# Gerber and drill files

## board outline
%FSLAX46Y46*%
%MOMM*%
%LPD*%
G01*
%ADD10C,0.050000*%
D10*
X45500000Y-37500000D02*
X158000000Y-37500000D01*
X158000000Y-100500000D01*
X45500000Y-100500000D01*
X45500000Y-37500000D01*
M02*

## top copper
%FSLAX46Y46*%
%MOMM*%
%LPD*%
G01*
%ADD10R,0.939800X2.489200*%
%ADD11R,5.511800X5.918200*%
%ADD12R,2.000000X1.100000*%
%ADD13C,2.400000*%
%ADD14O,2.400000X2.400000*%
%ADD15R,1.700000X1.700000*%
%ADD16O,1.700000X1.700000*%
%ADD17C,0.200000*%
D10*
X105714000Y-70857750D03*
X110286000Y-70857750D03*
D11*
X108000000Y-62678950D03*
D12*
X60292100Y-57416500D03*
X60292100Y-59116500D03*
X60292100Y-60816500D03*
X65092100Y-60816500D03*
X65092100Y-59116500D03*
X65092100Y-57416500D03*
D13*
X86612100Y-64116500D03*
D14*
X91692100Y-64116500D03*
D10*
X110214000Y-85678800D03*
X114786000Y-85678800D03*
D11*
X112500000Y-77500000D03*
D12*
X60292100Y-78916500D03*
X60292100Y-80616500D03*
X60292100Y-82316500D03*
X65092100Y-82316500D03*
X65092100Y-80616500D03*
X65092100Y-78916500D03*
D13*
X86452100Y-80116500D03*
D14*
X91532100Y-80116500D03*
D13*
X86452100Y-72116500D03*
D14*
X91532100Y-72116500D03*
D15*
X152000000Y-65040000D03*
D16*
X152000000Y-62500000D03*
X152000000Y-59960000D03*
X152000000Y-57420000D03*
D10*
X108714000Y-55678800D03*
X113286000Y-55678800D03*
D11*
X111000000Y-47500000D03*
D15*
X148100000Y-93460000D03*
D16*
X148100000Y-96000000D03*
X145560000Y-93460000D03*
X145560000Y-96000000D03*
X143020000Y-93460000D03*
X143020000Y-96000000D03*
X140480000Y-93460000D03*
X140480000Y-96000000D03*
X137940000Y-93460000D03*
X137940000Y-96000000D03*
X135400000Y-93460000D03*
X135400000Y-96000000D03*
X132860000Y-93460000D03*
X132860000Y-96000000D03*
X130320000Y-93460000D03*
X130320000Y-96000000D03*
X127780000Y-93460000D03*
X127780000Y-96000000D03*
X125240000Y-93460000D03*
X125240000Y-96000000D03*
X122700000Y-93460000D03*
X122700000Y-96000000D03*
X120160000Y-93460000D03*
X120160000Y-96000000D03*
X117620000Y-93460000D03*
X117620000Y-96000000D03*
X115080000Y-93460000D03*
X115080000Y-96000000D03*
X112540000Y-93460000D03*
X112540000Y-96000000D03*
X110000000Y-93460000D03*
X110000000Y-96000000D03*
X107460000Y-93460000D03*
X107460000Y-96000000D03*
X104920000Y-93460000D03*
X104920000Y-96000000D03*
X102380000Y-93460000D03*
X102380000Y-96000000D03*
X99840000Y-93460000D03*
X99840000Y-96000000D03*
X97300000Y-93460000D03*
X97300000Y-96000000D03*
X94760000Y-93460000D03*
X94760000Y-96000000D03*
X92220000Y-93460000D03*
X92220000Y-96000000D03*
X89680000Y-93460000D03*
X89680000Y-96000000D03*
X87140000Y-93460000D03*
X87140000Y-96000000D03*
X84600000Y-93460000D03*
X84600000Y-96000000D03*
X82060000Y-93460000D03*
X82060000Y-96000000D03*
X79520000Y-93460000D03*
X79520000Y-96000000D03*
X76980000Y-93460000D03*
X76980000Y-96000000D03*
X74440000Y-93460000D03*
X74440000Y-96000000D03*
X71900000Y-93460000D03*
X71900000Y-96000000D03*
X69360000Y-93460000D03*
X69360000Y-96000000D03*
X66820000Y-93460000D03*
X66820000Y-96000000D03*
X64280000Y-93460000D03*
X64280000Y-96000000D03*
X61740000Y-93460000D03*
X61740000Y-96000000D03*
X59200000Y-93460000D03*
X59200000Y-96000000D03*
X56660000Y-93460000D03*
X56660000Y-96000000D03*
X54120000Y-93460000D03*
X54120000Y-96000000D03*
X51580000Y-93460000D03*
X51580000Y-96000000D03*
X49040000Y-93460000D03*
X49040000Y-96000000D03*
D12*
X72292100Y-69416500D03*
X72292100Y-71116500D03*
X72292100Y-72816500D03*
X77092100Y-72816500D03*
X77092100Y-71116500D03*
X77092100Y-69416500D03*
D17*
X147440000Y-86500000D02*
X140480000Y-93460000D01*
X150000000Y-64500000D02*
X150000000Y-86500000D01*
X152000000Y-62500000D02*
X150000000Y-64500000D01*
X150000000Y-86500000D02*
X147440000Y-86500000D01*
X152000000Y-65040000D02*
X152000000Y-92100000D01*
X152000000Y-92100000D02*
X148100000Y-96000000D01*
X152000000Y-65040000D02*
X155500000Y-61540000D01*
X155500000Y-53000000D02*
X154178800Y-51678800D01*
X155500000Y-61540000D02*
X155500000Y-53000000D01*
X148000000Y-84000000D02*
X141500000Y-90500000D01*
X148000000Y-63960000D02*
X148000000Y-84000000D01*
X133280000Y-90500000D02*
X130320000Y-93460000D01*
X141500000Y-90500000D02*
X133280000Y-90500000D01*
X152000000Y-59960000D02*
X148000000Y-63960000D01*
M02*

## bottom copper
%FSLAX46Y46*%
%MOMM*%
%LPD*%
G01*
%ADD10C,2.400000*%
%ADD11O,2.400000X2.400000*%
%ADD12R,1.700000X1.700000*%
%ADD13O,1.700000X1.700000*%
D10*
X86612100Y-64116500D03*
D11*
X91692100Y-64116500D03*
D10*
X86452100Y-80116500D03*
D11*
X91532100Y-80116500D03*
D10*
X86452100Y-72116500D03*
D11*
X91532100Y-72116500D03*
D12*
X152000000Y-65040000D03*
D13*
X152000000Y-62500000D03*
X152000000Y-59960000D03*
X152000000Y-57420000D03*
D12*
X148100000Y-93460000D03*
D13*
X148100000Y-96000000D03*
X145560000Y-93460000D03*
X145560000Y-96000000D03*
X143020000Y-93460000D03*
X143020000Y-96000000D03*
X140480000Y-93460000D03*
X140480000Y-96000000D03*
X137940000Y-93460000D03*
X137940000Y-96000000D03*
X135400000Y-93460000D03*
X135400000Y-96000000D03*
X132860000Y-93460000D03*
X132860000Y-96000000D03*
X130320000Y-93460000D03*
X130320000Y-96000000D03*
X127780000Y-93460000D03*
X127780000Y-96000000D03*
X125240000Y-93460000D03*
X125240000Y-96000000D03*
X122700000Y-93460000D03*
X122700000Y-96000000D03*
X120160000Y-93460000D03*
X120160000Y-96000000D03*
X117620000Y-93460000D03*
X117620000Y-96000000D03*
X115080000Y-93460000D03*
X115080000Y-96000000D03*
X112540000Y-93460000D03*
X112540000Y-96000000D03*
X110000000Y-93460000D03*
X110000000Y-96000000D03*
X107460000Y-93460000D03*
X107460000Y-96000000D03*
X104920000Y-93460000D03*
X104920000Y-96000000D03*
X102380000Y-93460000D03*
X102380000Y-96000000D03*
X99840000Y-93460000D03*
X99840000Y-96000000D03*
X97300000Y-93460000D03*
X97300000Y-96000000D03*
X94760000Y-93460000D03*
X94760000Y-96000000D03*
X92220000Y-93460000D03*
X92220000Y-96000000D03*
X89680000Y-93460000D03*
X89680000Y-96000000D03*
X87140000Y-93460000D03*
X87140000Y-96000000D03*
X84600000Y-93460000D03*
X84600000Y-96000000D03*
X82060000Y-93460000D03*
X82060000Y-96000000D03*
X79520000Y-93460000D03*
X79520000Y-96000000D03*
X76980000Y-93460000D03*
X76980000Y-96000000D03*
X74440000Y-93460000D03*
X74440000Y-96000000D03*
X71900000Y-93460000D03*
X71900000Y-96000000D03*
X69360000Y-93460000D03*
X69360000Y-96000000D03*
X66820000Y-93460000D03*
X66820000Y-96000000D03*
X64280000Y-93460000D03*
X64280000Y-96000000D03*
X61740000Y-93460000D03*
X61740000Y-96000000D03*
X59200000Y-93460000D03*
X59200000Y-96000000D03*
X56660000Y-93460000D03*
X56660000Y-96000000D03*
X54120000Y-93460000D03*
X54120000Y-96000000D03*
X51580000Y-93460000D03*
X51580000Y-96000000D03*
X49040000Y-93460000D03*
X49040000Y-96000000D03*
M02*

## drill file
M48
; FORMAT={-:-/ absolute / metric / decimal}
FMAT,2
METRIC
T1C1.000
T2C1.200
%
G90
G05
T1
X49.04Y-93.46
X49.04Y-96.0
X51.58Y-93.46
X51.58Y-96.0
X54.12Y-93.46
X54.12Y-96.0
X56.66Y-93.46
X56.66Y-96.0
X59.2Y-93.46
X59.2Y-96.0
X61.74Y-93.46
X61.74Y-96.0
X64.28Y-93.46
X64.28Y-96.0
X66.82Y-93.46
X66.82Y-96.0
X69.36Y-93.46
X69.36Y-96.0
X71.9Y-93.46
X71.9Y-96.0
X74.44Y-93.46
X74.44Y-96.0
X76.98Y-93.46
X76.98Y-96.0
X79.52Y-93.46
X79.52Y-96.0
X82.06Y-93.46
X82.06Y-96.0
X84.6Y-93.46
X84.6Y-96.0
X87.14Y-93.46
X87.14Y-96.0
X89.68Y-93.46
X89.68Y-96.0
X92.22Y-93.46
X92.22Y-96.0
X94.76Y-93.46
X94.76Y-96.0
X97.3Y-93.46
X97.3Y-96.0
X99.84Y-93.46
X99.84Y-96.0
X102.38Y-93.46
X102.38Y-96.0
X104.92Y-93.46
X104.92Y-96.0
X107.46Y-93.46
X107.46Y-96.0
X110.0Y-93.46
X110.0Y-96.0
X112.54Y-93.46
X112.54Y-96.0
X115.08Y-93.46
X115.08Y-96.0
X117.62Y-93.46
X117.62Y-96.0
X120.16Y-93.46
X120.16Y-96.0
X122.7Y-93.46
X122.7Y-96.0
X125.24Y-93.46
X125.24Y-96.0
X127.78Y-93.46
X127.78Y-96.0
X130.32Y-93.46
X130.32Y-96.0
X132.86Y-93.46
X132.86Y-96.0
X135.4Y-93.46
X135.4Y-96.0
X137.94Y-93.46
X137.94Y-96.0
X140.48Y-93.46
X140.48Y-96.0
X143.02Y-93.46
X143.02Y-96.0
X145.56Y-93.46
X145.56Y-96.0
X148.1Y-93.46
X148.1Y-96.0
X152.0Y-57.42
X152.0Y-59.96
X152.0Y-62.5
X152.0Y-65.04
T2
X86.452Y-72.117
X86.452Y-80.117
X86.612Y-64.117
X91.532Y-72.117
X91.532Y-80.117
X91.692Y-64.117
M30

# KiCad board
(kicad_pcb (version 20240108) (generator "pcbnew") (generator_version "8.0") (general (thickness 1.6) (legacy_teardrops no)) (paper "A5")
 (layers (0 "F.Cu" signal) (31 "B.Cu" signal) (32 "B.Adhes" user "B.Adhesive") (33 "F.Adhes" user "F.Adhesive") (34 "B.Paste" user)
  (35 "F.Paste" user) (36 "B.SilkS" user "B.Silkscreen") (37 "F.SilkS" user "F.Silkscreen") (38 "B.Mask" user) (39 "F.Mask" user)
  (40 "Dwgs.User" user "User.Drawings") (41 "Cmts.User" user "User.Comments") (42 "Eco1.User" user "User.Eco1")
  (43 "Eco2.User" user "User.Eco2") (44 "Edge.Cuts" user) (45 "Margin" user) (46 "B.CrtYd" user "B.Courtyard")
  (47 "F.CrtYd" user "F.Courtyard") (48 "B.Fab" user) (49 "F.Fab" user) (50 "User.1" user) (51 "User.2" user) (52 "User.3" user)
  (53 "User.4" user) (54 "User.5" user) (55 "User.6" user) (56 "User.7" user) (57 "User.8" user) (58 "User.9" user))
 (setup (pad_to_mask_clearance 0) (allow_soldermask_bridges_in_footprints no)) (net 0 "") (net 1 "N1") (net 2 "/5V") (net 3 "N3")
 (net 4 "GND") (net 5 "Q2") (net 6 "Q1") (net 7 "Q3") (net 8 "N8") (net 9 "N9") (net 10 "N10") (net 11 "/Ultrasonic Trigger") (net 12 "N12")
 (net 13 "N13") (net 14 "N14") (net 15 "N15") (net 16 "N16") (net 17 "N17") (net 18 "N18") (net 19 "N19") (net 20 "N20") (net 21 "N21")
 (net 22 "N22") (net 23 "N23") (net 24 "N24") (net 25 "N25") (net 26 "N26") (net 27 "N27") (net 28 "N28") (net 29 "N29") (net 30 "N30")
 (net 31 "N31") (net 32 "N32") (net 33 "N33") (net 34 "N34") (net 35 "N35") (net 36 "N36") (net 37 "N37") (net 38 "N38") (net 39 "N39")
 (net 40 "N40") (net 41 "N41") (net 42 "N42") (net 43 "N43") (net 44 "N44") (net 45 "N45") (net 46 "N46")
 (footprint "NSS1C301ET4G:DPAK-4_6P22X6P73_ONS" (layer "F.Cu") (at 108 64.44425)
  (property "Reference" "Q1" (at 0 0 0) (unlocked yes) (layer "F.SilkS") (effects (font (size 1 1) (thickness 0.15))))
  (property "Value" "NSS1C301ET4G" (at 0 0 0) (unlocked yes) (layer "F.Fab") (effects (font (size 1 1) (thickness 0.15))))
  (pad "1" smd rect (at -2.286 6.4135) (size 0.9398 2.4892) (layers "F.Cu" "F.Paste" "F.Mask") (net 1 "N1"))
  (pad "2" smd rect (at 2.286 6.4135) (size 0.9398 2.4892) (layers "F.Cu" "F.Paste" "F.Mask") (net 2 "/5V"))
  (pad "3" smd rect (at 0 -1.7653) (size 5.5118 5.9182) (layers "F.Cu" "F.Paste" "F.Mask") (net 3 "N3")))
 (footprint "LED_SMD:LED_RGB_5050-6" (layer "F.Cu") (at 62.6921 59.1165)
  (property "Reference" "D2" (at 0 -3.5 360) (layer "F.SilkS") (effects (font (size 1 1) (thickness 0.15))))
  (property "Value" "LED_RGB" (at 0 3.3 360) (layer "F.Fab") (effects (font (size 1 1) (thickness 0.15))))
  (pad "1" smd rect (at -2.4 -1.7 90) (size 1.1 2) (layers "F.Cu" "F.Paste" "F.Mask") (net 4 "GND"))
  (pad "2" smd rect (at -2.4 0 90) (size 1.1 2) (layers "F.Cu" "F.Paste" "F.Mask") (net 4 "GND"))
  (pad "3" smd rect (at -2.4 1.7 90) (size 1.1 2) (layers "F.Cu" "F.Paste" "F.Mask") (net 4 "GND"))
  (pad "4" smd rect (at 2.4 1.7 90) (size 1.1 2) (layers "F.Cu" "F.Paste" "F.Mask") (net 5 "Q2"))
  (pad "5" smd rect (at 2.4 0 90) (size 1.1 2) (layers "F.Cu" "F.Paste" "F.Mask") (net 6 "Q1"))
  (pad "6" smd rect (at 2.4 -1.7 90) (size 1.1 2) (layers "F.Cu" "F.Paste" "F.Mask") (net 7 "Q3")))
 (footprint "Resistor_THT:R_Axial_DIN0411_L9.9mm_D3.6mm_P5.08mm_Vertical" (layer "F.Cu") (at 86.6121 64.1165)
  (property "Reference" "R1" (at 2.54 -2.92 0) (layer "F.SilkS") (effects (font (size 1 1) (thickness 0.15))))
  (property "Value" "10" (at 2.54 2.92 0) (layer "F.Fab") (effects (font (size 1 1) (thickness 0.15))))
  (pad "1" thru_hole circle (at 0 0) (size 2.4 2.4) (drill 1.2) (layers "*.Cu" "*.Mask") (remove_unused_layers no) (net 7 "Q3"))
  (pad "2" thru_hole oval (at 5.08 0) (size 2.4 2.4) (drill 1.2) (layers "*.Cu" "*.Mask") (remove_unused_layers no) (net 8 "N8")))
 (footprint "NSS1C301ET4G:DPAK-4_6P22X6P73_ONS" (layer "F.Cu") (at 112.5 79.2653)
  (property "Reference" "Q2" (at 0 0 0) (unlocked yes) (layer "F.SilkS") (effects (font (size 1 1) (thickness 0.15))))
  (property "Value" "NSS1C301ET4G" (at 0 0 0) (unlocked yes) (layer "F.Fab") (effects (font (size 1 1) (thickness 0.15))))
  (pad "1" smd rect (at -2.286 6.4135) (size 0.9398 2.4892) (layers "F.Cu" "F.Paste" "F.Mask") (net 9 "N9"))
  (pad "2" smd rect (at 2.286 6.4135) (size 0.9398 2.4892) (layers "F.Cu" "F.Paste" "F.Mask") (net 2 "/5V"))
  (pad "3" smd rect (at 0 -1.7653) (size 5.5118 5.9182) (layers "F.Cu" "F.Paste" "F.Mask") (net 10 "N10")))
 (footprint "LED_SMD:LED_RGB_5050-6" (layer "F.Cu") (at 62.6921 80.6165)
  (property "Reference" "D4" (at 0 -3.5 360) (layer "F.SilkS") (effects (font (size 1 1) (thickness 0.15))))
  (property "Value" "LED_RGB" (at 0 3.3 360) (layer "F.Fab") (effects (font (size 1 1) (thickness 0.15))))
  (pad "1" smd rect (at -2.4 -1.7 90) (size 1.1 2) (layers "F.Cu" "F.Paste" "F.Mask") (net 4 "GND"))
  (pad "2" smd rect (at -2.4 0 90) (size 1.1 2) (layers "F.Cu" "F.Paste" "F.Mask") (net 4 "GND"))
  (pad "3" smd rect (at -2.4 1.7 90) (size 1.1 2) (layers "F.Cu" "F.Paste" "F.Mask") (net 4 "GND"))
  (pad "4" smd rect (at 2.4 1.7 90) (size 1.1 2) (layers "F.Cu" "F.Paste" "F.Mask") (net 5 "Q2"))
  (pad "5" smd rect (at 2.4 0 90) (size 1.1 2) (layers "F.Cu" "F.Paste" "F.Mask") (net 6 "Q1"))
  (pad "6" smd rect (at 2.4 -1.7 90) (size 1.1 2) (layers "F.Cu" "F.Paste" "F.Mask") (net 7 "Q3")))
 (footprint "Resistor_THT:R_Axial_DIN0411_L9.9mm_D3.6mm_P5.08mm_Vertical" (layer "F.Cu") (at 86.4521 80.1165)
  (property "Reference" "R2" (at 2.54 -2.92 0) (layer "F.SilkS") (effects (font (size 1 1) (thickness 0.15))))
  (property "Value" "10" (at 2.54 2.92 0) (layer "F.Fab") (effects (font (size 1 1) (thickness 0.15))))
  (pad "1" thru_hole circle (at 0 0) (size 2.4 2.4) (drill 1.2) (layers "*.Cu" "*.Mask") (remove_unused_layers no) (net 5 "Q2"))
  (pad "2" thru_hole oval (at 5.08 0) (size 2.4 2.4) (drill 1.2) (layers "*.Cu" "*.Mask") (remove_unused_layers no) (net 10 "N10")))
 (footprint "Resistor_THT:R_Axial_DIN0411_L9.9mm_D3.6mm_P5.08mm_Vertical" (layer "F.Cu") (at 86.4521 72.1165)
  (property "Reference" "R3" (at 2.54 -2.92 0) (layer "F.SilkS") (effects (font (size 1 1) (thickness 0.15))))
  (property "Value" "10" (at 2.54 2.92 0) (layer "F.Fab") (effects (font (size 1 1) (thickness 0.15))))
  (pad "1" thru_hole circle (at 0 0) (size 2.4 2.4) (drill 1.2) (layers "*.Cu" "*.Mask") (remove_unused_layers no) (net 6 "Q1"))
  (pad "2" thru_hole oval (at 5.08 0) (size 2.4 2.4) (drill 1.2) (layers "*.Cu" "*.Mask") (remove_unused_layers no) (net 3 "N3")))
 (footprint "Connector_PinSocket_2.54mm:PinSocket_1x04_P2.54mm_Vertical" (layer "F.Cu") (at 152 65.04 180)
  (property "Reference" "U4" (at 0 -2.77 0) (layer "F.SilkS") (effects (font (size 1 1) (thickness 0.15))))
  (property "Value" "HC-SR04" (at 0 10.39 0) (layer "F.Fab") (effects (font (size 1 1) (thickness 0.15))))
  (pad "1" thru_hole rect (at 0 0 180) (size 1.7 1.7) (drill 1) (layers "*.Cu" "*.Mask") (remove_unused_layers no) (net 2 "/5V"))
  (pad "2" thru_hole oval (at 0 2.54 180) (size 1.7 1.7) (drill 1) (layers "*.Cu" "*.Mask") (remove_unused_layers no)
   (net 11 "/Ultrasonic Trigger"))
  (pad "3" thru_hole oval (at 0 5.08 180) (size 1.7 1.7) (drill 1) (layers "*.Cu" "*.Mask") (remove_unused_layers no) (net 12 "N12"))
  (pad "4" thru_hole oval (at 0 7.62 180) (size 1.7 1.7) (drill 1) (layers "*.Cu" "*.Mask") (remove_unused_layers no) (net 4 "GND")))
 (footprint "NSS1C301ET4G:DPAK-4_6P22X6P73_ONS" (layer "F.Cu") (at 111 49.2653)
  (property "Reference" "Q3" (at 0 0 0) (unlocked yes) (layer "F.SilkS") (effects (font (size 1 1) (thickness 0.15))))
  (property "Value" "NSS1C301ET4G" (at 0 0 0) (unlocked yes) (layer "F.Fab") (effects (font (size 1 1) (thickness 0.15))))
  (pad "1" smd rect (at -2.286 6.4135) (size 0.9398 2.4892) (layers "F.Cu" "F.Paste" "F.Mask") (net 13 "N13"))
  (pad "2" smd rect (at 2.286 6.4135) (size 0.9398 2.4892) (layers "F.Cu" "F.Paste" "F.Mask") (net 2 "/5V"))
  (pad "3" smd rect (at 0 -1.7653) (size 5.5118 5.9182) (layers "F.Cu" "F.Paste" "F.Mask") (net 8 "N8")))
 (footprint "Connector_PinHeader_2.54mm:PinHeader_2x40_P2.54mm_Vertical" (layer "F.Cu") (at 148.1 93.46 -90)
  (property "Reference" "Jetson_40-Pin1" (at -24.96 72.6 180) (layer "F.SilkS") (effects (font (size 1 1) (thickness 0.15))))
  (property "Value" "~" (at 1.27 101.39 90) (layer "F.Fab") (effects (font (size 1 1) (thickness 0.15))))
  (pad "1" thru_hole rect (at 0 0 270) (size 1.7 1.7) (drill 1) (layers "*.Cu" "*.Mask") (remove_unused_layers no) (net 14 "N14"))
  (pad "2" thru_hole oval (at 2.54 0 270) (size 1.7 1.7) (drill 1) (layers "*.Cu" "*.Mask") (remove_unused_layers no) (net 2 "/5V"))
  (pad "3" thru_hole oval (at 0 2.54 270) (size 1.7 1.7) (drill 1) (layers "*.Cu" "*.Mask") (remove_unused_layers no) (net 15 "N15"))
  (pad "4" thru_hole oval (at 2.54 2.54 270) (size 1.7 1.7) (drill 1) (layers "*.Cu" "*.Mask") (remove_unused_layers no) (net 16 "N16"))
  (pad "5" thru_hole oval (at 0 5.08 270) (size 1.7 1.7) (drill 1) (layers "*.Cu" "*.Mask") (remove_unused_layers no) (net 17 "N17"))
  (pad "6" thru_hole oval (at 2.54 5.08 270) (size 1.7 1.7) (drill 1) (layers "*.Cu" "*.Mask") (remove_unused_layers no) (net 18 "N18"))
  (pad "7" thru_hole oval (at 0 7.62 270) (size 1.7 1.7) (drill 1) (layers "*.Cu" "*.Mask") (remove_unused_layers no)
   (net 11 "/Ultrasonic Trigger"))
  (pad "8" thru_hole oval (at 2.54 7.62 270) (size 1.7 1.7) (drill 1) (layers "*.Cu" "*.Mask") (remove_unused_layers no) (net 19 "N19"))
  (pad "9" thru_hole oval (at 0 10.16 270) (size 1.7 1.7) (drill 1) (layers "*.Cu" "*.Mask") (remove_unused_layers no) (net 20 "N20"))
  (pad "10" thru_hole oval (at 2.54 10.16 270) (size 1.7 1.7) (drill 1) (layers "*.Cu" "*.Mask") (remove_unused_layers no) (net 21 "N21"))
  (pad "11" thru_hole oval (at 0 12.7 270) (size 1.7 1.7) (drill 1) (layers "*.Cu" "*.Mask") (remove_unused_layers no) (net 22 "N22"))
  (pad "12" thru_hole oval (at 2.54 12.7 270) (size 1.7 1.7) (drill 1) (layers "*.Cu" "*.Mask") (remove_unused_layers no) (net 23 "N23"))
  (pad "13" thru_hole oval (at 0 15.24 270) (size 1.7 1.7) (drill 1) (layers "*.Cu" "*.Mask") (remove_unused_layers no) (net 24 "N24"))
  (pad "14" thru_hole oval (at 2.54 15.24 270) (size 1.7 1.7) (drill 1) (layers "*.Cu" "*.Mask") (remove_unused_layers no) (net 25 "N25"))
  (pad "15" thru_hole oval (at 0 17.78 270) (size 1.7 1.7) (drill 1) (layers "*.Cu" "*.Mask") (remove_unused_layers no) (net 12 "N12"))
  (pad "16" thru_hole oval (at 2.54 17.78 270) (size 1.7 1.7) (drill 1) (layers "*.Cu" "*.Mask") (remove_unused_layers no) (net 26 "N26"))
  (pad "17" thru_hole oval (at 0 20.32 270) (size 1.7 1.7) (drill 1) (layers "*.Cu" "*.Mask") (remove_unused_layers no) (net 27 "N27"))
  (pad "18" thru_hole oval (at 2.54 20.32 270) (size 1.7 1.7) (drill 1) (layers "*.Cu" "*.Mask") (remove_unused_layers no) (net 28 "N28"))
  (pad "19" thru_hole oval (at 0 22.86 270) (size 1.7 1.7) (drill 1) (layers "*.Cu" "*.Mask") (remove_unused_layers no) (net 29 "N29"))
  (pad "20" thru_hole oval (at 2.54 22.86 270) (size 1.7 1.7) (drill 1) (layers "*.Cu" "*.Mask") (remove_unused_layers no) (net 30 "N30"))
  (pad "21" thru_hole oval (at 0 25.4 270) (size 1.7 1.7) (drill 1) (layers "*.Cu" "*.Mask") (remove_unused_layers no) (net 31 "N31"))
  (pad "22" thru_hole oval (at 2.54 25.4 270) (size 1.7 1.7) (drill 1) (layers "*.Cu" "*.Mask") (remove_unused_layers no) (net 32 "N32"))
  (pad "23" thru_hole oval (at 0 27.94 270) (size 1.7 1.7) (drill 1) (layers "*.Cu" "*.Mask") (remove_unused_layers no) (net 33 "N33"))
  (pad "24" thru_hole oval (at 2.54 27.94 270) (size 1.7 1.7) (drill 1) (layers "*.Cu" "*.Mask") (remove_unused_layers no) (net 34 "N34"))
  (pad "25" thru_hole oval (at 0 30.48 270) (size 1.7 1.7) (drill 1) (layers "*.Cu" "*.Mask") (remove_unused_layers no) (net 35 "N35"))
  (pad "26" thru_hole oval (at 2.54 30.48 270) (size 1.7 1.7) (drill 1) (layers "*.Cu" "*.Mask") (remove_unused_layers no) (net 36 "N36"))
  (pad "27" thru_hole oval (at 0 33.02 270) (size 1.7 1.7) (drill 1) (layers "*.Cu" "*.Mask") (remove_unused_layers no) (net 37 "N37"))
  (pad "28" thru_hole oval (at 2.54 33.02 270) (size 1.7 1.7) (drill 1) (layers "*.Cu" "*.Mask") (remove_unused_layers no) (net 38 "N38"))
  (pad "29" thru_hole oval (at 0 35.56 270) (size 1.7 1.7) (drill 1) (layers "*.Cu" "*.Mask") (remove_unused_layers no) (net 13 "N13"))
  (pad "30" thru_hole oval (at 2.54 35.56 270) (size 1.7 1.7) (drill 1) (layers "*.Cu" "*.Mask") (remove_unused_layers no) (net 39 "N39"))
  (pad "31" thru_hole oval (at 0 38.1 270) (size 1.7 1.7) (drill 1) (layers "*.Cu" "*.Mask") (remove_unused_layers no) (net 9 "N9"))
  (pad "32" thru_hole oval (at 2.54 38.1 270) (size 1.7 1.7) (drill 1) (layers "*.Cu" "*.Mask") (remove_unused_layers no) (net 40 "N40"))
  (pad "33" thru_hole oval (at 0 40.64 270) (size 1.7 1.7) (drill 1) (layers "*.Cu" "*.Mask") (remove_unused_layers no) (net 1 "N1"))
  (pad "34" thru_hole oval (at 2.54 40.64 270) (size 1.7 1.7) (drill 1) (layers "*.Cu" "*.Mask") (remove_unused_layers no) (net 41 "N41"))
  (pad "35" thru_hole oval (at 0 43.18 270) (size 1.7 1.7) (drill 1) (layers "*.Cu" "*.Mask") (remove_unused_layers no) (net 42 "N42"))
  (pad "36" thru_hole oval (at 2.54 43.18 270) (size 1.7 1.7) (drill 1) (layers "*.Cu" "*.Mask") (remove_unused_layers no) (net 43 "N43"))
  (pad "37" thru_hole oval (at 0 45.72 270) (size 1.7 1.7) (drill 1) (layers "*.Cu" "*.Mask") (remove_unused_layers no) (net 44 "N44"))
  (pad "38" thru_hole oval (at 2.54 45.72 270) (size 1.7 1.7) (drill 1) (layers "*.Cu" "*.Mask") (remove_unused_layers no) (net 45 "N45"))
  (pad "39" thru_hole oval (at 0 48.26 270) (size 1.7 1.7) (drill 1) (layers "*.Cu" "*.Mask") (remove_unused_layers no) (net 4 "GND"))
  (pad "40" thru_hole oval (at 2.54 48.26 270) (size 1.7 1.7) (drill 1) (layers "*.Cu" "*.Mask") (remove_unused_layers no) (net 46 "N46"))
  (pad "41" thru_hole oval (at 0 50.8 270) (size 1.7 1.7) (drill 1) (layers "*.Cu" "*.Mask") (remove_unused_layers no))
  (pad "42" thru_hole oval (at 2.54 50.8 270) (size 1.7 1.7) (drill 1) (layers "*.Cu" "*.Mask") (remove_unused_layers no))
  (pad "43" thru_hole oval (at 0 53.34 270) (size 1.7 1.7) (drill 1) (layers "*.Cu" "*.Mask") (remove_unused_layers no))
  (pad "44" thru_hole oval (at 2.54 53.34 270) (size 1.7 1.7) (drill 1) (layers "*.Cu" "*.Mask") (remove_unused_layers no))
  (pad "45" thru_hole oval (at 0 55.88 270) (size 1.7 1.7) (drill 1) (layers "*.Cu" "*.Mask") (remove_unused_layers no))
  (pad "46" thru_hole oval (at 2.54 55.88 270) (size 1.7 1.7) (drill 1) (layers "*.Cu" "*.Mask") (remove_unused_layers no))
  (pad "47" thru_hole oval (at 0 58.42 270) (size 1.7 1.7) (drill 1) (layers "*.Cu" "*.Mask") (remove_unused_layers no))
  (pad "48" thru_hole oval (at 2.54 58.42 270) (size 1.7 1.7) (drill 1) (layers "*.Cu" "*.Mask") (remove_unused_layers no))
  (pad "49" thru_hole oval (at 0 60.96 270) (size 1.7 1.7) (drill 1) (layers "*.Cu" "*.Mask") (remove_unused_layers no))
  (pad "50" thru_hole oval (at 2.54 60.96 270) (size 1.7 1.7) (drill 1) (layers "*.Cu" "*.Mask") (remove_unused_layers no))
  (pad "51" thru_hole oval (at 0 63.5 270) (size 1.7 1.7) (drill 1) (layers "*.Cu" "*.Mask") (remove_unused_layers no))
  (pad "52" thru_hole oval (at 2.54 63.5 270) (size 1.7 1.7) (drill 1) (layers "*.Cu" "*.Mask") (remove_unused_layers no))
  (pad "53" thru_hole oval (at 0 66.04 270) (size 1.7 1.7) (drill 1) (layers "*.Cu" "*.Mask") (remove_unused_layers no))
  (pad "54" thru_hole oval (at 2.54 66.04 270) (size 1.7 1.7) (drill 1) (layers "*.Cu" "*.Mask") (remove_unused_layers no))
  (pad "55" thru_hole oval (at 0 68.58 270) (size 1.7 1.7) (drill 1) (layers "*.Cu" "*.Mask") (remove_unused_layers no))
  (pad "56" thru_hole oval (at 2.54 68.58 270) (size 1.7 1.7) (drill 1) (layers "*.Cu" "*.Mask") (remove_unused_layers no))
  (pad "57" thru_hole oval (at 0 71.12 270) (size 1.7 1.7) (drill 1) (layers "*.Cu" "*.Mask") (remove_unused_layers no))
  (pad "58" thru_hole oval (at 2.54 71.12 270) (size 1.7 1.7) (drill 1) (layers "*.Cu" "*.Mask") (remove_unused_layers no))
  (pad "59" thru_hole oval (at 0 73.66 270) (size 1.7 1.7) (drill 1) (layers "*.Cu" "*.Mask") (remove_unused_layers no))
  (pad "60" thru_hole oval (at 2.54 73.66 270) (size 1.7 1.7) (drill 1) (layers "*.Cu" "*.Mask") (remove_unused_layers no))
  (pad "61" thru_hole oval (at 0 76.2 270) (size 1.7 1.7) (drill 1) (layers "*.Cu" "*.Mask") (remove_unused_layers no))
  (pad "62" thru_hole oval (at 2.54 76.2 270) (size 1.7 1.7) (drill 1) (layers "*.Cu" "*.Mask") (remove_unused_layers no))
  (pad "63" thru_hole oval (at 0 78.74 270) (size 1.7 1.7) (drill 1) (layers "*.Cu" "*.Mask") (remove_unused_layers no))
  (pad "64" thru_hole oval (at 2.54 78.74 270) (size 1.7 1.7) (drill 1) (layers "*.Cu" "*.Mask") (remove_unused_layers no))
  (pad "65" thru_hole oval (at 0 81.28 270) (size 1.7 1.7) (drill 1) (layers "*.Cu" "*.Mask") (remove_unused_layers no))
  (pad "66" thru_hole oval (at 2.54 81.28 270) (size 1.7 1.7) (drill 1) (layers "*.Cu" "*.Mask") (remove_unused_layers no))
  (pad "67" thru_hole oval (at 0 83.82 270) (size 1.7 1.7) (drill 1) (layers "*.Cu" "*.Mask") (remove_unused_layers no))
  (pad "68" thru_hole oval (at 2.54 83.82 270) (size 1.7 1.7) (drill 1) (layers "*.Cu" "*.Mask") (remove_unused_layers no))
  (pad "69" thru_hole oval (at 0 86.36 270) (size 1.7 1.7) (drill 1) (layers "*.Cu" "*.Mask") (remove_unused_layers no))
  (pad "70" thru_hole oval (at 2.54 86.36 270) (size 1.7 1.7) (drill 1) (layers "*.Cu" "*.Mask") (remove_unused_layers no))
  (pad "71" thru_hole oval (at 0 88.9 270) (size 1.7 1.7) (drill 1) (layers "*.Cu" "*.Mask") (remove_unused_layers no))
  (pad "72" thru_hole oval (at 2.54 88.9 270) (size 1.7 1.7) (drill 1) (layers "*.Cu" "*.Mask") (remove_unused_layers no))
  (pad "73" thru_hole oval (at 0 91.44 270) (size 1.7 1.7) (drill 1) (layers "*.Cu" "*.Mask") (remove_unused_layers no))
  (pad "74" thru_hole oval (at 2.54 91.44 270) (size 1.7 1.7) (drill 1) (layers "*.Cu" "*.Mask") (remove_unused_layers no))
  (pad "75" thru_hole oval (at 0 93.98 270) (size 1.7 1.7) (drill 1) (layers "*.Cu" "*.Mask") (remove_unused_layers no))
  (pad "76" thru_hole oval (at 2.54 93.98 270) (size 1.7 1.7) (drill 1) (layers "*.Cu" "*.Mask") (remove_unused_layers no))
  (pad "77" thru_hole oval (at 0 96.52 270) (size 1.7 1.7) (drill 1) (layers "*.Cu" "*.Mask") (remove_unused_layers no))
  (pad "78" thru_hole oval (at 2.54 96.52 270) (size 1.7 1.7) (drill 1) (layers "*.Cu" "*.Mask") (remove_unused_layers no))
  (pad "79" thru_hole oval (at 0 99.06 270) (size 1.7 1.7) (drill 1) (layers "*.Cu" "*.Mask") (remove_unused_layers no))
  (pad "80" thru_hole oval (at 2.54 99.06 270) (size 1.7 1.7) (drill 1) (layers "*.Cu" "*.Mask") (remove_unused_layers no)))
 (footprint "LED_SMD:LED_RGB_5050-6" (layer "F.Cu") (at 74.6921 71.1165)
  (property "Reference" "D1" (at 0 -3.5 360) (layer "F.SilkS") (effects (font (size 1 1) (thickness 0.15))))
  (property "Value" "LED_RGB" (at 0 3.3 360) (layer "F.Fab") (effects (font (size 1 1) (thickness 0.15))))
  (pad "1" smd rect (at -2.4 -1.7 90) (size 1.1 2) (layers "F.Cu" "F.Paste" "F.Mask") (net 4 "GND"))
  (pad "2" smd rect (at -2.4 0 90) (size 1.1 2) (layers "F.Cu" "F.Paste" "F.Mask") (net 4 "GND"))
  (pad "3" smd rect (at -2.4 1.7 90) (size 1.1 2) (layers "F.Cu" "F.Paste" "F.Mask") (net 4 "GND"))
  (pad "4" smd rect (at 2.4 1.7 90) (size 1.1 2) (layers "F.Cu" "F.Paste" "F.Mask") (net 5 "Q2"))
  (pad "5" smd rect (at 2.4 0 90) (size 1.1 2) (layers "F.Cu" "F.Paste" "F.Mask") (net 6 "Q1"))
  (pad "6" smd rect (at 2.4 -1.7 90) (size 1.1 2) (layers "F.Cu" "F.Paste" "F.Mask") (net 7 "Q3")))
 (gr_rect (start 45.5 37.5) (end 158 100.5) (stroke (width 0.05) (type default)) (fill none) (layer "Edge.Cuts"))
 (segment (start 147.44 86.5) (end 140.48 93.46) (width 0.2) (layer "F.Cu") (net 11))
 (segment (start 150 64.5) (end 150 86.5) (width 0.2) (layer "F.Cu") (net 11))
 (segment (start 152 62.5) (end 150 64.5) (width 0.2) (layer "F.Cu") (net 11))
 (segment (start 150 86.5) (end 147.44 86.5) (width 0.2) (layer "F.Cu") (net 11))
 (segment (start 152 65.04) (end 152 92.1) (width 0.2) (layer "F.Cu") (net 2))
 (segment (start 152 92.1) (end 148.1 96) (width 0.2) (layer "F.Cu") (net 2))
 (segment (start 152 65.04) (end 155.5 61.54) (width 0.2) (layer "F.Cu") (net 2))
 (segment (start 155.5 53) (end 154.1788 51.6788) (width 0.2) (layer "F.Cu") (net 2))
 (segment (start 155.5 61.54) (end 155.5 53) (width 0.2) (layer "F.Cu") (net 2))
 (segment (start 148 84) (end 141.5 90.5) (width 0.2) (layer "F.Cu") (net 12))
 (segment (start 148 63.96) (end 148 84) (width 0.2) (layer "F.Cu") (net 12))
 (segment (start 133.28 90.5) (end 130.32 93.46) (width 0.2) (layer "F.Cu") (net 12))
 (segment (start 141.5 90.5) (end 133.28 90.5) (width 0.2) (layer "F.Cu") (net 12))
 (segment (start 152 59.96) (end 148 63.96) (width 0.2) (layer "F.Cu") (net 12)))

